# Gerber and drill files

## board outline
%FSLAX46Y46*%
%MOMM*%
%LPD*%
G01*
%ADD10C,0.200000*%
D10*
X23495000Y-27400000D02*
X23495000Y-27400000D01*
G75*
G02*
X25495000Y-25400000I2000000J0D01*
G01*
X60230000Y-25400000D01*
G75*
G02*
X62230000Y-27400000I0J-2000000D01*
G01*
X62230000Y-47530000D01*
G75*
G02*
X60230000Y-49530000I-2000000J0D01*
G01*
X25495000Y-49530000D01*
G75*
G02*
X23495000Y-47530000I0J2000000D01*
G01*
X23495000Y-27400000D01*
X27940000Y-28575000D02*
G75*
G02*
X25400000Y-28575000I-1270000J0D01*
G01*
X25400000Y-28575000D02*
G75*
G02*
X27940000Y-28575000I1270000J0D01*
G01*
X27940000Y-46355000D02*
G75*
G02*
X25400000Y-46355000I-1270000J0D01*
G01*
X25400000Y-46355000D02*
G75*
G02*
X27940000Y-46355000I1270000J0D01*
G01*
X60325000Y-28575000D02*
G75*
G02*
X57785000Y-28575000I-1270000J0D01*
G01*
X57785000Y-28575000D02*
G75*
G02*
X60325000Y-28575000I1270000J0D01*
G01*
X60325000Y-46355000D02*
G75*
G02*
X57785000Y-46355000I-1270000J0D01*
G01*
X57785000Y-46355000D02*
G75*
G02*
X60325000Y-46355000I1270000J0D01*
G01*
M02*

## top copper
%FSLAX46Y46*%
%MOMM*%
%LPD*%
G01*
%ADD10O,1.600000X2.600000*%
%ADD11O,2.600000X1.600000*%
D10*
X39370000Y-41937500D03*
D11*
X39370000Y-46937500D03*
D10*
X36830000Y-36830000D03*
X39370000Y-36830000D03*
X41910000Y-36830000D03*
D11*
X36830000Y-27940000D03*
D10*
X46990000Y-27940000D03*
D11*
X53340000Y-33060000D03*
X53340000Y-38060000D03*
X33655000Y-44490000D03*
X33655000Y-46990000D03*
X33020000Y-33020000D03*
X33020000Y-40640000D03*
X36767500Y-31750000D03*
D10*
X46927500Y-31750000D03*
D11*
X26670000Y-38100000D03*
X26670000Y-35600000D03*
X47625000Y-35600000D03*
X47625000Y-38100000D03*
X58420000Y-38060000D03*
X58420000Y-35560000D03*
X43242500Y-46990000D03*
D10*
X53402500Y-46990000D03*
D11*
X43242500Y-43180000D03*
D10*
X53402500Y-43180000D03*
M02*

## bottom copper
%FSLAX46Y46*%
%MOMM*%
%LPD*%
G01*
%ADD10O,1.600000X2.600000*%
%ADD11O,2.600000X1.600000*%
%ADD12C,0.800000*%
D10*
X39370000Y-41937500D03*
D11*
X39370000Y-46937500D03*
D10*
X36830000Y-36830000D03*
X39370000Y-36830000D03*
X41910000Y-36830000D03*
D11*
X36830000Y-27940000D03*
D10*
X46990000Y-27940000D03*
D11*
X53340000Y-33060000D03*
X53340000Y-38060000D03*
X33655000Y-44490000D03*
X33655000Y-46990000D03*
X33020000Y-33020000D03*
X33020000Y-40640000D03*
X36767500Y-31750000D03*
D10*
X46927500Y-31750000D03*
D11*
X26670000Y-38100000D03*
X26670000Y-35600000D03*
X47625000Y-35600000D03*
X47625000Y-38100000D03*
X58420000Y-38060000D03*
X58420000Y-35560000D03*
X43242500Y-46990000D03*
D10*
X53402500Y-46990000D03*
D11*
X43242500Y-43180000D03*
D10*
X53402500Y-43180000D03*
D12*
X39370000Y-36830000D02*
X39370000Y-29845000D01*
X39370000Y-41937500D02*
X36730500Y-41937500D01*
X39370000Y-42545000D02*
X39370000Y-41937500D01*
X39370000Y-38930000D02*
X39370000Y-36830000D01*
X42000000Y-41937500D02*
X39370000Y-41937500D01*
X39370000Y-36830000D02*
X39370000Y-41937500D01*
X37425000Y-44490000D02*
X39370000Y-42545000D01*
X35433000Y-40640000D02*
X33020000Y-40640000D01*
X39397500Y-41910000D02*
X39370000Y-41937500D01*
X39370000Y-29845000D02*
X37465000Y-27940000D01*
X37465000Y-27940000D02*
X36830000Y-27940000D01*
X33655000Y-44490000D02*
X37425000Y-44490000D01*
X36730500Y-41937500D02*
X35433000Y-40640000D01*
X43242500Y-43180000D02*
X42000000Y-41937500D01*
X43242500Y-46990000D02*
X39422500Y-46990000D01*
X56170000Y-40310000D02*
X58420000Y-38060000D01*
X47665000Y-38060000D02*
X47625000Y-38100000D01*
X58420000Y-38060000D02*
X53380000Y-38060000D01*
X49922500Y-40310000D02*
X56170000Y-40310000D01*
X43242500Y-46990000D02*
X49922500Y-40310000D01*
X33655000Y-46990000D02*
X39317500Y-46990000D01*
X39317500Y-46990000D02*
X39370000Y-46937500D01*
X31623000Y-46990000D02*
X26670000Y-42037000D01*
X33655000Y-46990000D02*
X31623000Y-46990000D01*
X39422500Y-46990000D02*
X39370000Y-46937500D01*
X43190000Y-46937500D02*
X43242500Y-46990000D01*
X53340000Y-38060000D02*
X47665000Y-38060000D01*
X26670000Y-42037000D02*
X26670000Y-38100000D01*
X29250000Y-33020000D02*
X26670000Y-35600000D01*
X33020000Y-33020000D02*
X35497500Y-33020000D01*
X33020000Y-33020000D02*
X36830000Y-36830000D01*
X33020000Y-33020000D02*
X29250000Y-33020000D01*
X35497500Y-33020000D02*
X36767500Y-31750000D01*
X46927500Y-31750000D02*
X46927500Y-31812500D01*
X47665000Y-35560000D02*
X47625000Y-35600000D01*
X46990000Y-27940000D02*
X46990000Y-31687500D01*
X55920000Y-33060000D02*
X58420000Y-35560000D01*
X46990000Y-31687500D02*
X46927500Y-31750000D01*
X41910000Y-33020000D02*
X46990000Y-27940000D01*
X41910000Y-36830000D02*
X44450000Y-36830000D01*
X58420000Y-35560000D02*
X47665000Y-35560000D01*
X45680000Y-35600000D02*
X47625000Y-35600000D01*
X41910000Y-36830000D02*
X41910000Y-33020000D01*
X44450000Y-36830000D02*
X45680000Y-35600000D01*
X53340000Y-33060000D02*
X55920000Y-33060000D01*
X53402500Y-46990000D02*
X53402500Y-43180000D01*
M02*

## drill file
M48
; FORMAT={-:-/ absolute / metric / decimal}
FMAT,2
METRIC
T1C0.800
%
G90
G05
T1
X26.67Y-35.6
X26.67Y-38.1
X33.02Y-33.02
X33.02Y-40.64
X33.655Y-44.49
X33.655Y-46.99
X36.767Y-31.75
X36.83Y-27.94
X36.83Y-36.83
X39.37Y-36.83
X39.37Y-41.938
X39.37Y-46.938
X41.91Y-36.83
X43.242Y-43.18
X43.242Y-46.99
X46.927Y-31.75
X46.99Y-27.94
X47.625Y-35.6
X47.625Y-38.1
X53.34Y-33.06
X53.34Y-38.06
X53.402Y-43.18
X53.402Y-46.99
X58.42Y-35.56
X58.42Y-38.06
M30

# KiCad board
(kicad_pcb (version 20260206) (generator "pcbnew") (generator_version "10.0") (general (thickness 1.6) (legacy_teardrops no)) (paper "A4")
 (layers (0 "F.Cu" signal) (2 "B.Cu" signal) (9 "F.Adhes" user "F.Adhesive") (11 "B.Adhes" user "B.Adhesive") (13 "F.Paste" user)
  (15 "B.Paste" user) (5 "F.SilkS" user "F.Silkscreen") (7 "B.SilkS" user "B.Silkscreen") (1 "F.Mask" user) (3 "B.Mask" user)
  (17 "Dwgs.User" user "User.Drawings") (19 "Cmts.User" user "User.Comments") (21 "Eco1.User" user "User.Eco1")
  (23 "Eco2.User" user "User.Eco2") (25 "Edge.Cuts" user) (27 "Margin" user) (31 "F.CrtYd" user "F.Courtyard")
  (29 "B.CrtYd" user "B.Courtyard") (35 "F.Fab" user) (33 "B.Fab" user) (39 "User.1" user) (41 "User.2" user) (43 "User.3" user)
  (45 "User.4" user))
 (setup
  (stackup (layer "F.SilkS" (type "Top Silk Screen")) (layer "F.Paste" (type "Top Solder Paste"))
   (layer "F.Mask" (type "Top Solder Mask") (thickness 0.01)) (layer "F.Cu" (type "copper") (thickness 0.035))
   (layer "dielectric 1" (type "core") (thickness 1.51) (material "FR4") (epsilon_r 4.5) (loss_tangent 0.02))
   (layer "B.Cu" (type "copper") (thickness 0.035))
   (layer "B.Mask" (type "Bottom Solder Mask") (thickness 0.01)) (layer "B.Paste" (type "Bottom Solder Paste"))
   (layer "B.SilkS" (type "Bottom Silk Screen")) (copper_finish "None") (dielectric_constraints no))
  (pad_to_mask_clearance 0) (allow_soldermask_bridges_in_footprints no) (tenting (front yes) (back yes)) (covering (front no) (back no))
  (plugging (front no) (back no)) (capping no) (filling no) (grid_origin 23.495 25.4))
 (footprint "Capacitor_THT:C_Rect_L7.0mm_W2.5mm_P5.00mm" (layer "F.Cu") (at 39.37 41.9375 -90)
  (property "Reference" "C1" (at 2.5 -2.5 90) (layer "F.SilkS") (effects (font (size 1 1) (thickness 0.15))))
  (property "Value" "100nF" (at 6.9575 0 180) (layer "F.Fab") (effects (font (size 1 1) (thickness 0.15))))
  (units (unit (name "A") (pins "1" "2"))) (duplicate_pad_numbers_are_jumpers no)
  (pad "1" thru_hole oval (at 0 0) (size 1.6 2.6) (drill 0.8) (layers "*.Cu" "*.Mask") (remove_unused_layers no) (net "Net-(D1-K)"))
  (pad "2" thru_hole oval (at 5 0 270) (size 1.6 2.6) (drill 0.8) (layers "*.Cu" "*.Mask") (remove_unused_layers no) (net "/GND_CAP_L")))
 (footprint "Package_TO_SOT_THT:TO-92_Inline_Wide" (layer "F.Cu") (at 36.83 36.83)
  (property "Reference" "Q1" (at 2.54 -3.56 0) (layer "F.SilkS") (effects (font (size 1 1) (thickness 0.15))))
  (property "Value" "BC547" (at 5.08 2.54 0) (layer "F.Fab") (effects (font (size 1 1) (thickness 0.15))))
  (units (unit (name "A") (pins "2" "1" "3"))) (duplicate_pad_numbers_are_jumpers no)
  (pad "1" thru_hole oval (at 0 0) (size 1.6 2.6) (drill 0.8) (layers "*.Cu" "*.Mask") (remove_unused_layers no) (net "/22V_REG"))
  (pad "2" thru_hole oval (at 2.54 0) (size 1.6 2.6) (drill 0.8) (layers "*.Cu" "*.Mask") (remove_unused_layers no) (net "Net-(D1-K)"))
  (pad "3" thru_hole oval (at 5.08 0) (size 1.6 2.6) (drill 0.8) (layers "*.Cu" "*.Mask") (remove_unused_layers no)
   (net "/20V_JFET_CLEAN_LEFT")))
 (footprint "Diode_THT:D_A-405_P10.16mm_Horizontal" (layer "F.Cu") (at 36.83 27.94)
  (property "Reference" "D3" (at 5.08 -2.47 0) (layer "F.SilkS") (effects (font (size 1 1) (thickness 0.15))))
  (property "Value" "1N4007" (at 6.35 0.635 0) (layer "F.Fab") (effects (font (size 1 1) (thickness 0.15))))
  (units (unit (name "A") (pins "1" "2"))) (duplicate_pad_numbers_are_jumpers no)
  (pad "1" thru_hole oval (at 0 0 90) (size 1.6 2.6) (drill 0.8) (layers "*.Cu" "*.Mask") (remove_unused_layers no) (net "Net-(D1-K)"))
  (pad "2" thru_hole oval (at 10.16 0) (size 1.6 2.6) (drill 0.8) (layers "*.Cu" "*.Mask") (remove_unused_layers no)
   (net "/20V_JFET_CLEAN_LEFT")))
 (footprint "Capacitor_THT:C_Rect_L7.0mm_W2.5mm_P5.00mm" (layer "F.Cu") (at 53.34 33.06 -90)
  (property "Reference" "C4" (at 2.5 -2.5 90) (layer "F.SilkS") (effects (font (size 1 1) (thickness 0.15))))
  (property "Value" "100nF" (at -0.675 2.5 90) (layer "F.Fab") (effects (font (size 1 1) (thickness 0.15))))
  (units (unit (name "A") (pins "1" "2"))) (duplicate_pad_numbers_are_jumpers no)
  (pad "1" thru_hole oval (at 0 0 270) (size 1.6 2.6) (drill 0.8) (layers "*.Cu" "*.Mask") (remove_unused_layers no)
   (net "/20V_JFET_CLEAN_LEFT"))
  (pad "2" thru_hole oval (at 5 0 270) (size 1.6 2.6) (drill 0.8) (layers "*.Cu" "*.Mask") (remove_unused_layers no) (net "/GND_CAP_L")))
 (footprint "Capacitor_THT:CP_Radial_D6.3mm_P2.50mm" (layer "F.Cu") (at 33.655 44.49 -90)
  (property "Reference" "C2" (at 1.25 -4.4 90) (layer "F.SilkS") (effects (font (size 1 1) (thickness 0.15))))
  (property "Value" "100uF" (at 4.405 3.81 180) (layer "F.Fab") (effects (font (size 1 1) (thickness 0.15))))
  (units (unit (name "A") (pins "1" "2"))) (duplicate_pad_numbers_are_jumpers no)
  (pad "1" thru_hole oval (at 0 0 270) (size 1.6 2.6) (drill 0.8) (layers "*.Cu" "*.Mask") (remove_unused_layers no) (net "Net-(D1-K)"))
  (pad "2" thru_hole oval (at 2.5 0 270) (size 1.6 2.6) (drill 0.8) (layers "*.Cu" "*.Mask") (remove_unused_layers no) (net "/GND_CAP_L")))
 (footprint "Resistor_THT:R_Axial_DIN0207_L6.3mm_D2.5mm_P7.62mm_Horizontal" (layer "F.Cu") (at 33.02 33.02 -90)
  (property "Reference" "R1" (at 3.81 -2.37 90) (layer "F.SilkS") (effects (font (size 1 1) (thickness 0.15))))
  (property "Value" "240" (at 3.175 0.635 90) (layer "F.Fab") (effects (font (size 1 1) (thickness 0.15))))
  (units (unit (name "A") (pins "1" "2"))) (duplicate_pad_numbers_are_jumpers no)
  (pad "1" thru_hole oval (at 0 0 270) (size 1.6 2.6) (drill 0.8) (layers "*.Cu" "*.Mask") (remove_unused_layers no) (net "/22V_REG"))
  (pad "2" thru_hole oval (at 7.62 0 270) (size 1.6 2.6) (drill 0.8) (layers "*.Cu" "*.Mask") (remove_unused_layers no) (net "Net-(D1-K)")))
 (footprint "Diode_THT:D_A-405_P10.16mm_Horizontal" (layer "F.Cu") (at 36.7675 31.75)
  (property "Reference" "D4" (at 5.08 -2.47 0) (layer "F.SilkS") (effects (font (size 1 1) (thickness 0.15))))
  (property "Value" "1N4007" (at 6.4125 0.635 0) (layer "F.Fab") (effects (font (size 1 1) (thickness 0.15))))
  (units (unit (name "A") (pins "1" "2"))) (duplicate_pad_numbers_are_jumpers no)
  (pad "1" thru_hole oval (at 0 0 90) (size 1.6 2.6) (drill 0.8) (layers "*.Cu" "*.Mask") (remove_unused_layers no) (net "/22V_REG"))
  (pad "2" thru_hole oval (at 10.16 0) (size 1.6 2.6) (drill 0.8) (layers "*.Cu" "*.Mask") (remove_unused_layers no)
   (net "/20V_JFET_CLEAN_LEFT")))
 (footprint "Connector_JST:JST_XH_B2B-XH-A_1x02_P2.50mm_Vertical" (layer "F.Cu") (at 26.67 38.1 90)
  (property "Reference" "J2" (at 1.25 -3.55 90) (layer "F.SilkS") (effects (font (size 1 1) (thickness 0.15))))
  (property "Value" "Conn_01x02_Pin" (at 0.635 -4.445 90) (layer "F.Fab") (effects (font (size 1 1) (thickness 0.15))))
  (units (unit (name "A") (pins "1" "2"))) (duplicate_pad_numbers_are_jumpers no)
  (pad "1" thru_hole oval (at 0 0 90) (size 1.6 2.6) (drill 0.8) (layers "*.Cu" "*.Mask") (remove_unused_layers no) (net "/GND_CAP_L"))
  (pad "2" thru_hole oval (at 2.5 0 90) (size 1.6 2.6) (drill 0.8) (layers "*.Cu" "*.Mask") (remove_unused_layers no) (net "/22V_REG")))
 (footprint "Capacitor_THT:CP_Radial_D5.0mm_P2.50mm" (layer "F.Cu") (at 47.625 35.6 -90)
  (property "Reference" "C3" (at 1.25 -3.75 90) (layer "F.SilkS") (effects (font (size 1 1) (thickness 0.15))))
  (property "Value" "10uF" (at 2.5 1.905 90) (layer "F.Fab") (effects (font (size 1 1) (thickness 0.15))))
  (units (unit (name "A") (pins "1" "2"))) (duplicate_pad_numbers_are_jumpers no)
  (pad "1" thru_hole oval (at 0 0 270) (size 1.6 2.6) (drill 0.8) (layers "*.Cu" "*.Mask") (remove_unused_layers no)
   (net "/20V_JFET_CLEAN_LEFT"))
  (pad "2" thru_hole oval (at 2.5 0 270) (size 1.6 2.6) (drill 0.8) (layers "*.Cu" "*.Mask") (remove_unused_layers no) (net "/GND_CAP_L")))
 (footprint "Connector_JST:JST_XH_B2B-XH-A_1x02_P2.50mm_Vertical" (layer "F.Cu") (at 58.42 38.06 90)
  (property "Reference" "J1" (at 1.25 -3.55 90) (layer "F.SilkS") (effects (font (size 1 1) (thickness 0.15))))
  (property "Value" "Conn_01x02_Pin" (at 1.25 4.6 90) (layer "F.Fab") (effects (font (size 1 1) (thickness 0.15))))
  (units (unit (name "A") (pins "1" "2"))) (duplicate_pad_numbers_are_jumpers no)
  (pad "1" thru_hole oval (at 0 0 90) (size 1.6 2.6) (drill 0.8) (layers "*.Cu" "*.Mask") (remove_unused_layers no) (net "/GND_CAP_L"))
  (pad "2" thru_hole oval (at 2.5 0 90) (size 1.6 2.6) (drill 0.8) (layers "*.Cu" "*.Mask") (remove_unused_layers no)
   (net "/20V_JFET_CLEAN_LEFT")))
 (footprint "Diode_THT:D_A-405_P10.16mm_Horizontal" (layer "F.Cu") (at 43.2425 46.99)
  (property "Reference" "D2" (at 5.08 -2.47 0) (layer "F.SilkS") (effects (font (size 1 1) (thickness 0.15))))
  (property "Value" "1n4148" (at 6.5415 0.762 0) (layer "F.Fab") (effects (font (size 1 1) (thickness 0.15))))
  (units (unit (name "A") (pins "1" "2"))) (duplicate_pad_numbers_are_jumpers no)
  (pad "1" thru_hole oval (at 0 0 90) (size 1.6 2.6) (drill 0.8) (layers "*.Cu" "*.Mask") (remove_unused_layers no) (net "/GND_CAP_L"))
  (pad "2" thru_hole oval (at 10.16 0) (size 1.6 2.6) (drill 0.8) (layers "*.Cu" "*.Mask") (remove_unused_layers no) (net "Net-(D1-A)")))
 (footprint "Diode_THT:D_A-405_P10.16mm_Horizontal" (layer "F.Cu") (at 43.2425 43.18)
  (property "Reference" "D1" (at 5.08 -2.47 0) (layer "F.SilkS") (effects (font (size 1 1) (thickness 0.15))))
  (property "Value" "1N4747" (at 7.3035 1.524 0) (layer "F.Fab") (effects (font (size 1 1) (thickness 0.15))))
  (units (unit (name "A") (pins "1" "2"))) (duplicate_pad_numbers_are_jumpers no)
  (pad "1" thru_hole oval (at 0 0 90) (size 1.6 2.6) (drill 0.8) (layers "*.Cu" "*.Mask") (remove_unused_layers no) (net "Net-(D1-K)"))
  (pad "2" thru_hole oval (at 10.16 0) (size 1.6 2.6) (drill 0.8) (layers "*.Cu" "*.Mask") (remove_unused_layers no) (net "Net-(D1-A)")))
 (gr_rect (start 23.495 25.4) (end 62.23 49.53) (radius 2) (stroke (width 0.2) (type solid)) (fill no) (layer "Edge.Cuts"))
 (gr_circle (center 26.67 28.575) (end 27.94 28.575) (stroke (width 0.2) (type solid)) (fill no) (layer "Edge.Cuts"))
 (gr_circle (center 26.67 46.355) (end 27.94 46.355) (stroke (width 0.2) (type solid)) (fill no) (layer "Edge.Cuts"))
 (gr_circle (center 59.055 28.575) (end 60.325 28.575) (stroke (width 0.2) (type solid)) (fill no) (layer "Edge.Cuts"))
 (gr_circle (center 59.055 46.355) (end 60.325 46.355) (stroke (width 0.2) (type solid)) (fill no) (layer "Edge.Cuts"))
 (segment (start 39.37 36.83) (end 39.37 29.845) (width 0.8) (layer "B.Cu") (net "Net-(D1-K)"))
 (segment (start 39.37 41.9375) (end 36.7305 41.9375) (width 0.8) (layer "B.Cu") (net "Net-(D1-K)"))
 (segment (start 39.37 42.545) (end 39.37 41.9375) (width 0.8) (layer "B.Cu") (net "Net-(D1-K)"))
 (segment (start 39.37 38.93) (end 39.37 36.83) (width 0.8) (layer "B.Cu") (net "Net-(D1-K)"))
 (segment (start 42 41.9375) (end 39.37 41.9375) (width 0.8) (layer "B.Cu") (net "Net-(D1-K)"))
 (segment (start 39.37 36.83) (end 39.37 41.9375) (width 0.8) (layer "B.Cu") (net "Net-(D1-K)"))
 (segment (start 37.425 44.49) (end 39.37 42.545) (width 0.8) (layer "B.Cu") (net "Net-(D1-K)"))
 (segment (start 35.433 40.64) (end 33.02 40.64) (width 0.8) (layer "B.Cu") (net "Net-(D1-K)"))
 (segment (start 39.3975 41.91) (end 39.37 41.9375) (width 0.8) (layer "B.Cu") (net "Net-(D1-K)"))
 (segment (start 39.37 29.845) (end 37.465 27.94) (width 0.8) (layer "B.Cu") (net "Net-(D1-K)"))
 (segment (start 37.465 27.94) (end 36.83 27.94) (width 0.8) (layer "B.Cu") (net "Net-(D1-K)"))
 (segment (start 33.655 44.49) (end 37.425 44.49) (width 0.8) (layer "B.Cu") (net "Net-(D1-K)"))
 (segment (start 36.7305 41.9375) (end 35.433 40.64) (width 0.8) (layer "B.Cu") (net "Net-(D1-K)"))
 (segment (start 43.2425 43.18) (end 42 41.9375) (width 0.8) (layer "B.Cu") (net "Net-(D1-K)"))
 (segment (start 43.2425 46.99) (end 39.4225 46.99) (width 0.8) (layer "B.Cu") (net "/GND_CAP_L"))
 (segment (start 56.17 40.31) (end 58.42 38.06) (width 0.8) (layer "B.Cu") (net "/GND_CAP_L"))
 (segment (start 47.665 38.06) (end 47.625 38.1) (width 0.8) (layer "B.Cu") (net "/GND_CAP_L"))
 (segment (start 58.42 38.06) (end 53.38 38.06) (width 0.8) (layer "B.Cu") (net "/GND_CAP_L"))
 (segment (start 49.9225 40.31) (end 56.17 40.31) (width 0.8) (layer "B.Cu") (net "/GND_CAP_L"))
 (segment (start 43.2425 46.99) (end 49.9225 40.31) (width 0.8) (layer "B.Cu") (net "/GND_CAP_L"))
 (segment (start 33.655 46.99) (end 39.3175 46.99) (width 0.8) (layer "B.Cu") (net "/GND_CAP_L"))
 (segment (start 39.3175 46.99) (end 39.37 46.9375) (width 0.8) (layer "B.Cu") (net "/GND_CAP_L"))
 (segment (start 31.623 46.99) (end 26.67 42.037) (width 0.8) (layer "B.Cu") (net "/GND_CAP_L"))
 (segment (start 33.655 46.99) (end 31.623 46.99) (width 0.8) (layer "B.Cu") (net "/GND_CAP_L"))
 (segment (start 39.4225 46.99) (end 39.37 46.9375) (width 0.8) (layer "B.Cu") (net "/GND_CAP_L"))
 (segment (start 43.19 46.9375) (end 43.2425 46.99) (width 0.8) (layer "B.Cu") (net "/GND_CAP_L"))
 (segment (start 53.34 38.06) (end 47.665 38.06) (width 0.8) (layer "B.Cu") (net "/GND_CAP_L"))
 (segment (start 26.67 42.037) (end 26.67 38.1) (width 0.8) (layer "B.Cu") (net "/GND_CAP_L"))
 (segment (start 29.25 33.02) (end 26.67 35.6) (width 0.8) (layer "B.Cu") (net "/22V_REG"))
 (segment (start 33.02 33.02) (end 35.4975 33.02) (width 0.8) (layer "B.Cu") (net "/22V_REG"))
 (segment (start 33.02 33.02) (end 36.83 36.83) (width 0.8) (layer "B.Cu") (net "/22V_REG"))
 (segment (start 33.02 33.02) (end 29.25 33.02) (width 0.8) (layer "B.Cu") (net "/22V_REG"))
 (segment (start 35.4975 33.02) (end 36.7675 31.75) (width 0.8) (layer "B.Cu") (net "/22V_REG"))
 (segment (start 46.9275 31.75) (end 46.9275 31.8125) (width 0.8) (layer "B.Cu") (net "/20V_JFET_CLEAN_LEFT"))
 (segment (start 47.665 35.56) (end 47.625 35.6) (width 0.8) (layer "B.Cu") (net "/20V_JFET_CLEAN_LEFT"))
 (segment (start 46.99 27.94) (end 46.99 31.6875) (width 0.8) (layer "B.Cu") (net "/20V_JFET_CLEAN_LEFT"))
 (segment (start 55.92 33.06) (end 58.42 35.56) (width 0.8) (layer "B.Cu") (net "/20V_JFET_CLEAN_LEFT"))
 (segment (start 46.99 31.6875) (end 46.9275 31.75) (width 0.8) (layer "B.Cu") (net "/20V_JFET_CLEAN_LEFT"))
 (segment (start 41.91 33.02) (end 46.99 27.94) (width 0.8) (layer "B.Cu") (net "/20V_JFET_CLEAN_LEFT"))
 (segment (start 41.91 36.83) (end 44.45 36.83) (width 0.8) (layer "B.Cu") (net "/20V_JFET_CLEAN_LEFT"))
 (segment (start 58.42 35.56) (end 47.665 35.56) (width 0.8) (layer "B.Cu") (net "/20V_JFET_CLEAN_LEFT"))
 (segment (start 45.68 35.6) (end 47.625 35.6) (width 0.8) (layer "B.Cu") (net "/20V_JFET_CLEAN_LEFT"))
 (segment (start 41.91 36.83) (end 41.91 33.02) (width 0.8) (layer "B.Cu") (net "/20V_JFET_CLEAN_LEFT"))
 (segment (start 44.45 36.83) (end 45.68 35.6) (width 0.8) (layer "B.Cu") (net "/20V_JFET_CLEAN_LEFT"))
 (segment (start 53.34 33.06) (end 55.92 33.06) (width 0.8) (layer "B.Cu") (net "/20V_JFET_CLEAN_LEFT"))
 (segment (start 53.4025 46.99) (end 53.4025 43.18) (width 0.8) (layer "B.Cu") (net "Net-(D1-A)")))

